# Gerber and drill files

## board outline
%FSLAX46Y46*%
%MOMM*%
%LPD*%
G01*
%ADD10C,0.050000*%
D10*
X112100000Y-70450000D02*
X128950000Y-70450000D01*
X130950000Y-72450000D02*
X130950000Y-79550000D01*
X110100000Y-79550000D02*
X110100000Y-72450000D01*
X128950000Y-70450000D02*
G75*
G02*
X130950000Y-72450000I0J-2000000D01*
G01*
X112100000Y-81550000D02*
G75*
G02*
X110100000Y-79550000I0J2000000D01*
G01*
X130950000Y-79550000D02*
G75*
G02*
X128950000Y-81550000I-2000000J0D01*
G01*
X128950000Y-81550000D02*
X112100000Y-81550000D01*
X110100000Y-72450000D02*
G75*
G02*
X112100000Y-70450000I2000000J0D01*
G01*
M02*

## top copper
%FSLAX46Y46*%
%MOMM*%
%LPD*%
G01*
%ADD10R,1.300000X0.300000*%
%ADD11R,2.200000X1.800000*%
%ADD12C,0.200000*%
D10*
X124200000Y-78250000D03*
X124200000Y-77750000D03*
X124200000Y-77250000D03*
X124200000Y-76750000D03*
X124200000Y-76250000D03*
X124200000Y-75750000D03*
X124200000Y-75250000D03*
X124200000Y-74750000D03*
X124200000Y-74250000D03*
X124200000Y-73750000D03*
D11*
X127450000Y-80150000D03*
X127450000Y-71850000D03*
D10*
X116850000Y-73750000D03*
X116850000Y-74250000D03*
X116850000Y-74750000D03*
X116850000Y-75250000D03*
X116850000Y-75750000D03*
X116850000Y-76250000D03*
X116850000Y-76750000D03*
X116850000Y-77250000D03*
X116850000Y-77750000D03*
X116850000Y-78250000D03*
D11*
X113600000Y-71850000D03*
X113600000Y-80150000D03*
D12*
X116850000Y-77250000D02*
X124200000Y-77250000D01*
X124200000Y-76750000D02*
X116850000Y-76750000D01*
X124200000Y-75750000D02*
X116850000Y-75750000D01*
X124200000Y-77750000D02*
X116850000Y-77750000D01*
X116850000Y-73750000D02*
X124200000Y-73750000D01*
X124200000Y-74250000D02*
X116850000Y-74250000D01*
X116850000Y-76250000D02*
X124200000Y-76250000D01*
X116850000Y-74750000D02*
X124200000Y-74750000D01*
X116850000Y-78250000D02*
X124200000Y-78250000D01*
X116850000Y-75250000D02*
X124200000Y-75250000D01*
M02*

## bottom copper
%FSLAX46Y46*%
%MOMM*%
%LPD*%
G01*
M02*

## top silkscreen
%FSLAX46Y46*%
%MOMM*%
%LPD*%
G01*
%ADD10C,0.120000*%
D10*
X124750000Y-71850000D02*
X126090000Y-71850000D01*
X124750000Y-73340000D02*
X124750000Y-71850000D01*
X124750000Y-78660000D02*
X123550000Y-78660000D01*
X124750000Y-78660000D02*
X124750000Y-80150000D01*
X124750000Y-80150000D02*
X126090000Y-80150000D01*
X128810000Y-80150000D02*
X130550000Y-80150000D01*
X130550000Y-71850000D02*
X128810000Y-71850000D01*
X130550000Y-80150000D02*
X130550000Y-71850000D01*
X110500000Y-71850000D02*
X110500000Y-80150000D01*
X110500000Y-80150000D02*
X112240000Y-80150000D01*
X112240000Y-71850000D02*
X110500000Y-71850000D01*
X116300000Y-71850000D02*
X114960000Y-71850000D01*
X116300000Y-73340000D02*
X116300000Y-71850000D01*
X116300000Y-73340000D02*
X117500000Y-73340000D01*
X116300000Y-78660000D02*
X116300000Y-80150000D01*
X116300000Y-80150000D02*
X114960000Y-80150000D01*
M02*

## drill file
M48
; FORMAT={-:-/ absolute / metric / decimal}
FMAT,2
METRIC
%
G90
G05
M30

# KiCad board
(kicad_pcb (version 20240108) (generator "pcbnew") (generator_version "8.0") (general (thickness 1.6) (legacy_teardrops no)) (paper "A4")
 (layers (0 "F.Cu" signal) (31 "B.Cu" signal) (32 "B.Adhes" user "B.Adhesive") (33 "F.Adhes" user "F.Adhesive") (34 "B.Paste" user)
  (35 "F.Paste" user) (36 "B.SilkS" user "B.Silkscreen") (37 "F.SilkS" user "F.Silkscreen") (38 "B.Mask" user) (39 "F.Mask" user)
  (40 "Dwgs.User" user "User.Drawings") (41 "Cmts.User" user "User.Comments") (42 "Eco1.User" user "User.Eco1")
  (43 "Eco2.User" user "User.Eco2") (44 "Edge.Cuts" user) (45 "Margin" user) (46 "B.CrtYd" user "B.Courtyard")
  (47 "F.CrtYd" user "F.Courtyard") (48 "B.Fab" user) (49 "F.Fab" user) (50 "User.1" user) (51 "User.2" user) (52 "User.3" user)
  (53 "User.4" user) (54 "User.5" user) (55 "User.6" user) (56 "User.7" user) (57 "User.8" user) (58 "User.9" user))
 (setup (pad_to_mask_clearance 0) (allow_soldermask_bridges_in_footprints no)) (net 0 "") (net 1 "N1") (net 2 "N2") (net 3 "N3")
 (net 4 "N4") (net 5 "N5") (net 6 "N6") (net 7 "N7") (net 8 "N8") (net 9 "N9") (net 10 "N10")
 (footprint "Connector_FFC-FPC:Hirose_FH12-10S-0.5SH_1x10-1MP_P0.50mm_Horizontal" (layer "F.Cu") (at 126.05 76 90)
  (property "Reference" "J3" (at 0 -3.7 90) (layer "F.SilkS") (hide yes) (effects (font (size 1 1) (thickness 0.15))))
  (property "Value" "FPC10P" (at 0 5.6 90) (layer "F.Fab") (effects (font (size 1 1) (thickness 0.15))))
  (fp_line (start 4.15 -1.3) (end 4.15 0.04) (stroke (width 0.12) (type solid)) (layer "F.SilkS"))
  (fp_line (start 2.66 -1.3) (end 4.15 -1.3) (stroke (width 0.12) (type solid)) (layer "F.SilkS"))
  (fp_line (start -2.66 -1.3) (end -2.66 -2.5) (stroke (width 0.12) (type solid)) (layer "F.SilkS"))
  (fp_line (start -2.66 -1.3) (end -4.15 -1.3) (stroke (width 0.12) (type solid)) (layer "F.SilkS"))
  (fp_line (start -4.15 -1.3) (end -4.15 0.04) (stroke (width 0.12) (type solid)) (layer "F.SilkS"))
  (fp_line (start -4.15 2.76) (end -4.15 4.5) (stroke (width 0.12) (type solid)) (layer "F.SilkS"))
  (fp_line (start 4.15 4.5) (end 4.15 2.76) (stroke (width 0.12) (type solid)) (layer "F.SilkS"))
  (fp_line (start -4.15 4.5) (end 4.15 4.5) (stroke (width 0.12) (type solid)) (layer "F.SilkS"))
  (pad "1" smd rect (at -2.25 -1.85 90) (size 0.3 1.3) (layers "F.Cu" "F.Paste" "F.Mask") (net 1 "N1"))
  (pad "2" smd rect (at -1.75 -1.85 90) (size 0.3 1.3) (layers "F.Cu" "F.Paste" "F.Mask") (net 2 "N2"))
  (pad "3" smd rect (at -1.25 -1.85 90) (size 0.3 1.3) (layers "F.Cu" "F.Paste" "F.Mask") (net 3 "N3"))
  (pad "4" smd rect (at -0.75 -1.85 90) (size 0.3 1.3) (layers "F.Cu" "F.Paste" "F.Mask") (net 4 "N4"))
  (pad "5" smd rect (at -0.25 -1.85 90) (size 0.3 1.3) (layers "F.Cu" "F.Paste" "F.Mask") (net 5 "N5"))
  (pad "6" smd rect (at 0.25 -1.85 90) (size 0.3 1.3) (layers "F.Cu" "F.Paste" "F.Mask") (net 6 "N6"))
  (pad "7" smd rect (at 0.75 -1.85 90) (size 0.3 1.3) (layers "F.Cu" "F.Paste" "F.Mask") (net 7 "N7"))
  (pad "8" smd rect (at 1.25 -1.85 90) (size 0.3 1.3) (layers "F.Cu" "F.Paste" "F.Mask") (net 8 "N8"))
  (pad "9" smd rect (at 1.75 -1.85 90) (size 0.3 1.3) (layers "F.Cu" "F.Paste" "F.Mask") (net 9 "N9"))
  (pad "10" smd rect (at 2.25 -1.85 90) (size 0.3 1.3) (layers "F.Cu" "F.Paste" "F.Mask") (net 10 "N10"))
  (pad "MP" smd rect (at -4.15 1.4 90) (size 1.8 2.2) (layers "F.Cu" "F.Paste" "F.Mask"))
  (pad "MP" smd rect (at 4.15 1.4 90) (size 1.8 2.2) (layers "F.Cu" "F.Paste" "F.Mask")))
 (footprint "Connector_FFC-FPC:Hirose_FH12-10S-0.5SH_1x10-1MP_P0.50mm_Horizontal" (layer "F.Cu") (at 115 76 -90)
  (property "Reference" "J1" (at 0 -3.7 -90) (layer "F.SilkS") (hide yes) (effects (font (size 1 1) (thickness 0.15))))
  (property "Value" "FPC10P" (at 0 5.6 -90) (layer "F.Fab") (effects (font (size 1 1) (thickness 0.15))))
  (fp_line (start -4.15 4.5) (end 4.15 4.5) (stroke (width 0.12) (type solid)) (layer "F.SilkS"))
  (fp_line (start 4.15 4.5) (end 4.15 2.76) (stroke (width 0.12) (type solid)) (layer "F.SilkS"))
  (fp_line (start -4.15 2.76) (end -4.15 4.5) (stroke (width 0.12) (type solid)) (layer "F.SilkS"))
  (fp_line (start -4.15 -1.3) (end -4.15 0.04) (stroke (width 0.12) (type solid)) (layer "F.SilkS"))
  (fp_line (start -2.66 -1.3) (end -4.15 -1.3) (stroke (width 0.12) (type solid)) (layer "F.SilkS"))
  (fp_line (start -2.66 -1.3) (end -2.66 -2.5) (stroke (width 0.12) (type solid)) (layer "F.SilkS"))
  (fp_line (start 2.66 -1.3) (end 4.15 -1.3) (stroke (width 0.12) (type solid)) (layer "F.SilkS"))
  (fp_line (start 4.15 -1.3) (end 4.15 0.04) (stroke (width 0.12) (type solid)) (layer "F.SilkS"))
  (pad "1" smd rect (at -2.25 -1.85 270) (size 0.3 1.3) (layers "F.Cu" "F.Paste" "F.Mask") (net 10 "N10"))
  (pad "2" smd rect (at -1.75 -1.85 270) (size 0.3 1.3) (layers "F.Cu" "F.Paste" "F.Mask") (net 9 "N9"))
  (pad "3" smd rect (at -1.25 -1.85 270) (size 0.3 1.3) (layers "F.Cu" "F.Paste" "F.Mask") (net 8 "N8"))
  (pad "4" smd rect (at -0.75 -1.85 270) (size 0.3 1.3) (layers "F.Cu" "F.Paste" "F.Mask") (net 7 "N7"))
  (pad "5" smd rect (at -0.25 -1.85 270) (size 0.3 1.3) (layers "F.Cu" "F.Paste" "F.Mask") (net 6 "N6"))
  (pad "6" smd rect (at 0.25 -1.85 270) (size 0.3 1.3) (layers "F.Cu" "F.Paste" "F.Mask") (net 5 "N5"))
  (pad "7" smd rect (at 0.75 -1.85 270) (size 0.3 1.3) (layers "F.Cu" "F.Paste" "F.Mask") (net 4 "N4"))
  (pad "8" smd rect (at 1.25 -1.85 270) (size 0.3 1.3) (layers "F.Cu" "F.Paste" "F.Mask") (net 3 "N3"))
  (pad "9" smd rect (at 1.75 -1.85 270) (size 0.3 1.3) (layers "F.Cu" "F.Paste" "F.Mask") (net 2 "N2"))
  (pad "10" smd rect (at 2.25 -1.85 270) (size 0.3 1.3) (layers "F.Cu" "F.Paste" "F.Mask") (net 1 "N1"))
  (pad "MP" smd rect (at -4.15 1.4 270) (size 1.8 2.2) (layers "F.Cu" "F.Paste" "F.Mask"))
  (pad "MP" smd rect (at 4.15 1.4 270) (size 1.8 2.2) (layers "F.Cu" "F.Paste" "F.Mask")))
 (gr_line (start 112.1 70.45) (end 128.95 70.45) (stroke (width 0.05) (type default)) (layer "Edge.Cuts"))
 (gr_line (start 130.95 72.45) (end 130.95 79.55) (stroke (width 0.05) (type default)) (layer "Edge.Cuts"))
 (gr_line (start 110.1 79.55) (end 110.1 72.45) (stroke (width 0.05) (type default)) (layer "Edge.Cuts"))
 (gr_arc (start 128.95 70.45) (mid 130.364214 71.035786) (end 130.95 72.45) (stroke (width 0.05) (type default)) (layer "Edge.Cuts"))
 (gr_arc (start 112.1 81.55) (mid 110.685786 80.964214) (end 110.1 79.55) (stroke (width 0.05) (type default)) (layer "Edge.Cuts"))
 (gr_arc (start 130.95 79.55) (mid 130.364214 80.964214) (end 128.95 81.55) (stroke (width 0.05) (type default)) (layer "Edge.Cuts"))
 (gr_line (start 128.95 81.55) (end 112.1 81.55) (stroke (width 0.05) (type default)) (layer "Edge.Cuts"))
 (gr_arc (start 110.1 72.45) (mid 110.685786 71.035786) (end 112.1 70.45) (stroke (width 0.05) (type default)) (layer "Edge.Cuts"))
 (segment (start 116.85 77.25) (end 124.2 77.25) (width 0.2) (layer "F.Cu") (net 3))
 (segment (start 124.2 76.75) (end 116.85 76.75) (width 0.2) (layer "F.Cu") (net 4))
 (segment (start 124.2 75.75) (end 116.85 75.75) (width 0.2) (layer "F.Cu") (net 6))
 (segment (start 124.2 77.75) (end 116.85 77.75) (width 0.2) (layer "F.Cu") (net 2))
 (segment (start 116.85 73.75) (end 124.2 73.75) (width 0.2) (layer "F.Cu") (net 10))
 (segment (start 124.2 74.25) (end 116.85 74.25) (width 0.2) (layer "F.Cu") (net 9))
 (segment (start 116.85 76.25) (end 124.2 76.25) (width 0.2) (layer "F.Cu") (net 5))
 (segment (start 116.85 74.75) (end 124.2 74.75) (width 0.2) (layer "F.Cu") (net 8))
 (segment (start 116.85 78.25) (end 124.2 78.25) (width 0.2) (layer "F.Cu") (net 1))
 (segment (start 116.85 75.25) (end 124.2 75.25) (width 0.2) (layer "F.Cu") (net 7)))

